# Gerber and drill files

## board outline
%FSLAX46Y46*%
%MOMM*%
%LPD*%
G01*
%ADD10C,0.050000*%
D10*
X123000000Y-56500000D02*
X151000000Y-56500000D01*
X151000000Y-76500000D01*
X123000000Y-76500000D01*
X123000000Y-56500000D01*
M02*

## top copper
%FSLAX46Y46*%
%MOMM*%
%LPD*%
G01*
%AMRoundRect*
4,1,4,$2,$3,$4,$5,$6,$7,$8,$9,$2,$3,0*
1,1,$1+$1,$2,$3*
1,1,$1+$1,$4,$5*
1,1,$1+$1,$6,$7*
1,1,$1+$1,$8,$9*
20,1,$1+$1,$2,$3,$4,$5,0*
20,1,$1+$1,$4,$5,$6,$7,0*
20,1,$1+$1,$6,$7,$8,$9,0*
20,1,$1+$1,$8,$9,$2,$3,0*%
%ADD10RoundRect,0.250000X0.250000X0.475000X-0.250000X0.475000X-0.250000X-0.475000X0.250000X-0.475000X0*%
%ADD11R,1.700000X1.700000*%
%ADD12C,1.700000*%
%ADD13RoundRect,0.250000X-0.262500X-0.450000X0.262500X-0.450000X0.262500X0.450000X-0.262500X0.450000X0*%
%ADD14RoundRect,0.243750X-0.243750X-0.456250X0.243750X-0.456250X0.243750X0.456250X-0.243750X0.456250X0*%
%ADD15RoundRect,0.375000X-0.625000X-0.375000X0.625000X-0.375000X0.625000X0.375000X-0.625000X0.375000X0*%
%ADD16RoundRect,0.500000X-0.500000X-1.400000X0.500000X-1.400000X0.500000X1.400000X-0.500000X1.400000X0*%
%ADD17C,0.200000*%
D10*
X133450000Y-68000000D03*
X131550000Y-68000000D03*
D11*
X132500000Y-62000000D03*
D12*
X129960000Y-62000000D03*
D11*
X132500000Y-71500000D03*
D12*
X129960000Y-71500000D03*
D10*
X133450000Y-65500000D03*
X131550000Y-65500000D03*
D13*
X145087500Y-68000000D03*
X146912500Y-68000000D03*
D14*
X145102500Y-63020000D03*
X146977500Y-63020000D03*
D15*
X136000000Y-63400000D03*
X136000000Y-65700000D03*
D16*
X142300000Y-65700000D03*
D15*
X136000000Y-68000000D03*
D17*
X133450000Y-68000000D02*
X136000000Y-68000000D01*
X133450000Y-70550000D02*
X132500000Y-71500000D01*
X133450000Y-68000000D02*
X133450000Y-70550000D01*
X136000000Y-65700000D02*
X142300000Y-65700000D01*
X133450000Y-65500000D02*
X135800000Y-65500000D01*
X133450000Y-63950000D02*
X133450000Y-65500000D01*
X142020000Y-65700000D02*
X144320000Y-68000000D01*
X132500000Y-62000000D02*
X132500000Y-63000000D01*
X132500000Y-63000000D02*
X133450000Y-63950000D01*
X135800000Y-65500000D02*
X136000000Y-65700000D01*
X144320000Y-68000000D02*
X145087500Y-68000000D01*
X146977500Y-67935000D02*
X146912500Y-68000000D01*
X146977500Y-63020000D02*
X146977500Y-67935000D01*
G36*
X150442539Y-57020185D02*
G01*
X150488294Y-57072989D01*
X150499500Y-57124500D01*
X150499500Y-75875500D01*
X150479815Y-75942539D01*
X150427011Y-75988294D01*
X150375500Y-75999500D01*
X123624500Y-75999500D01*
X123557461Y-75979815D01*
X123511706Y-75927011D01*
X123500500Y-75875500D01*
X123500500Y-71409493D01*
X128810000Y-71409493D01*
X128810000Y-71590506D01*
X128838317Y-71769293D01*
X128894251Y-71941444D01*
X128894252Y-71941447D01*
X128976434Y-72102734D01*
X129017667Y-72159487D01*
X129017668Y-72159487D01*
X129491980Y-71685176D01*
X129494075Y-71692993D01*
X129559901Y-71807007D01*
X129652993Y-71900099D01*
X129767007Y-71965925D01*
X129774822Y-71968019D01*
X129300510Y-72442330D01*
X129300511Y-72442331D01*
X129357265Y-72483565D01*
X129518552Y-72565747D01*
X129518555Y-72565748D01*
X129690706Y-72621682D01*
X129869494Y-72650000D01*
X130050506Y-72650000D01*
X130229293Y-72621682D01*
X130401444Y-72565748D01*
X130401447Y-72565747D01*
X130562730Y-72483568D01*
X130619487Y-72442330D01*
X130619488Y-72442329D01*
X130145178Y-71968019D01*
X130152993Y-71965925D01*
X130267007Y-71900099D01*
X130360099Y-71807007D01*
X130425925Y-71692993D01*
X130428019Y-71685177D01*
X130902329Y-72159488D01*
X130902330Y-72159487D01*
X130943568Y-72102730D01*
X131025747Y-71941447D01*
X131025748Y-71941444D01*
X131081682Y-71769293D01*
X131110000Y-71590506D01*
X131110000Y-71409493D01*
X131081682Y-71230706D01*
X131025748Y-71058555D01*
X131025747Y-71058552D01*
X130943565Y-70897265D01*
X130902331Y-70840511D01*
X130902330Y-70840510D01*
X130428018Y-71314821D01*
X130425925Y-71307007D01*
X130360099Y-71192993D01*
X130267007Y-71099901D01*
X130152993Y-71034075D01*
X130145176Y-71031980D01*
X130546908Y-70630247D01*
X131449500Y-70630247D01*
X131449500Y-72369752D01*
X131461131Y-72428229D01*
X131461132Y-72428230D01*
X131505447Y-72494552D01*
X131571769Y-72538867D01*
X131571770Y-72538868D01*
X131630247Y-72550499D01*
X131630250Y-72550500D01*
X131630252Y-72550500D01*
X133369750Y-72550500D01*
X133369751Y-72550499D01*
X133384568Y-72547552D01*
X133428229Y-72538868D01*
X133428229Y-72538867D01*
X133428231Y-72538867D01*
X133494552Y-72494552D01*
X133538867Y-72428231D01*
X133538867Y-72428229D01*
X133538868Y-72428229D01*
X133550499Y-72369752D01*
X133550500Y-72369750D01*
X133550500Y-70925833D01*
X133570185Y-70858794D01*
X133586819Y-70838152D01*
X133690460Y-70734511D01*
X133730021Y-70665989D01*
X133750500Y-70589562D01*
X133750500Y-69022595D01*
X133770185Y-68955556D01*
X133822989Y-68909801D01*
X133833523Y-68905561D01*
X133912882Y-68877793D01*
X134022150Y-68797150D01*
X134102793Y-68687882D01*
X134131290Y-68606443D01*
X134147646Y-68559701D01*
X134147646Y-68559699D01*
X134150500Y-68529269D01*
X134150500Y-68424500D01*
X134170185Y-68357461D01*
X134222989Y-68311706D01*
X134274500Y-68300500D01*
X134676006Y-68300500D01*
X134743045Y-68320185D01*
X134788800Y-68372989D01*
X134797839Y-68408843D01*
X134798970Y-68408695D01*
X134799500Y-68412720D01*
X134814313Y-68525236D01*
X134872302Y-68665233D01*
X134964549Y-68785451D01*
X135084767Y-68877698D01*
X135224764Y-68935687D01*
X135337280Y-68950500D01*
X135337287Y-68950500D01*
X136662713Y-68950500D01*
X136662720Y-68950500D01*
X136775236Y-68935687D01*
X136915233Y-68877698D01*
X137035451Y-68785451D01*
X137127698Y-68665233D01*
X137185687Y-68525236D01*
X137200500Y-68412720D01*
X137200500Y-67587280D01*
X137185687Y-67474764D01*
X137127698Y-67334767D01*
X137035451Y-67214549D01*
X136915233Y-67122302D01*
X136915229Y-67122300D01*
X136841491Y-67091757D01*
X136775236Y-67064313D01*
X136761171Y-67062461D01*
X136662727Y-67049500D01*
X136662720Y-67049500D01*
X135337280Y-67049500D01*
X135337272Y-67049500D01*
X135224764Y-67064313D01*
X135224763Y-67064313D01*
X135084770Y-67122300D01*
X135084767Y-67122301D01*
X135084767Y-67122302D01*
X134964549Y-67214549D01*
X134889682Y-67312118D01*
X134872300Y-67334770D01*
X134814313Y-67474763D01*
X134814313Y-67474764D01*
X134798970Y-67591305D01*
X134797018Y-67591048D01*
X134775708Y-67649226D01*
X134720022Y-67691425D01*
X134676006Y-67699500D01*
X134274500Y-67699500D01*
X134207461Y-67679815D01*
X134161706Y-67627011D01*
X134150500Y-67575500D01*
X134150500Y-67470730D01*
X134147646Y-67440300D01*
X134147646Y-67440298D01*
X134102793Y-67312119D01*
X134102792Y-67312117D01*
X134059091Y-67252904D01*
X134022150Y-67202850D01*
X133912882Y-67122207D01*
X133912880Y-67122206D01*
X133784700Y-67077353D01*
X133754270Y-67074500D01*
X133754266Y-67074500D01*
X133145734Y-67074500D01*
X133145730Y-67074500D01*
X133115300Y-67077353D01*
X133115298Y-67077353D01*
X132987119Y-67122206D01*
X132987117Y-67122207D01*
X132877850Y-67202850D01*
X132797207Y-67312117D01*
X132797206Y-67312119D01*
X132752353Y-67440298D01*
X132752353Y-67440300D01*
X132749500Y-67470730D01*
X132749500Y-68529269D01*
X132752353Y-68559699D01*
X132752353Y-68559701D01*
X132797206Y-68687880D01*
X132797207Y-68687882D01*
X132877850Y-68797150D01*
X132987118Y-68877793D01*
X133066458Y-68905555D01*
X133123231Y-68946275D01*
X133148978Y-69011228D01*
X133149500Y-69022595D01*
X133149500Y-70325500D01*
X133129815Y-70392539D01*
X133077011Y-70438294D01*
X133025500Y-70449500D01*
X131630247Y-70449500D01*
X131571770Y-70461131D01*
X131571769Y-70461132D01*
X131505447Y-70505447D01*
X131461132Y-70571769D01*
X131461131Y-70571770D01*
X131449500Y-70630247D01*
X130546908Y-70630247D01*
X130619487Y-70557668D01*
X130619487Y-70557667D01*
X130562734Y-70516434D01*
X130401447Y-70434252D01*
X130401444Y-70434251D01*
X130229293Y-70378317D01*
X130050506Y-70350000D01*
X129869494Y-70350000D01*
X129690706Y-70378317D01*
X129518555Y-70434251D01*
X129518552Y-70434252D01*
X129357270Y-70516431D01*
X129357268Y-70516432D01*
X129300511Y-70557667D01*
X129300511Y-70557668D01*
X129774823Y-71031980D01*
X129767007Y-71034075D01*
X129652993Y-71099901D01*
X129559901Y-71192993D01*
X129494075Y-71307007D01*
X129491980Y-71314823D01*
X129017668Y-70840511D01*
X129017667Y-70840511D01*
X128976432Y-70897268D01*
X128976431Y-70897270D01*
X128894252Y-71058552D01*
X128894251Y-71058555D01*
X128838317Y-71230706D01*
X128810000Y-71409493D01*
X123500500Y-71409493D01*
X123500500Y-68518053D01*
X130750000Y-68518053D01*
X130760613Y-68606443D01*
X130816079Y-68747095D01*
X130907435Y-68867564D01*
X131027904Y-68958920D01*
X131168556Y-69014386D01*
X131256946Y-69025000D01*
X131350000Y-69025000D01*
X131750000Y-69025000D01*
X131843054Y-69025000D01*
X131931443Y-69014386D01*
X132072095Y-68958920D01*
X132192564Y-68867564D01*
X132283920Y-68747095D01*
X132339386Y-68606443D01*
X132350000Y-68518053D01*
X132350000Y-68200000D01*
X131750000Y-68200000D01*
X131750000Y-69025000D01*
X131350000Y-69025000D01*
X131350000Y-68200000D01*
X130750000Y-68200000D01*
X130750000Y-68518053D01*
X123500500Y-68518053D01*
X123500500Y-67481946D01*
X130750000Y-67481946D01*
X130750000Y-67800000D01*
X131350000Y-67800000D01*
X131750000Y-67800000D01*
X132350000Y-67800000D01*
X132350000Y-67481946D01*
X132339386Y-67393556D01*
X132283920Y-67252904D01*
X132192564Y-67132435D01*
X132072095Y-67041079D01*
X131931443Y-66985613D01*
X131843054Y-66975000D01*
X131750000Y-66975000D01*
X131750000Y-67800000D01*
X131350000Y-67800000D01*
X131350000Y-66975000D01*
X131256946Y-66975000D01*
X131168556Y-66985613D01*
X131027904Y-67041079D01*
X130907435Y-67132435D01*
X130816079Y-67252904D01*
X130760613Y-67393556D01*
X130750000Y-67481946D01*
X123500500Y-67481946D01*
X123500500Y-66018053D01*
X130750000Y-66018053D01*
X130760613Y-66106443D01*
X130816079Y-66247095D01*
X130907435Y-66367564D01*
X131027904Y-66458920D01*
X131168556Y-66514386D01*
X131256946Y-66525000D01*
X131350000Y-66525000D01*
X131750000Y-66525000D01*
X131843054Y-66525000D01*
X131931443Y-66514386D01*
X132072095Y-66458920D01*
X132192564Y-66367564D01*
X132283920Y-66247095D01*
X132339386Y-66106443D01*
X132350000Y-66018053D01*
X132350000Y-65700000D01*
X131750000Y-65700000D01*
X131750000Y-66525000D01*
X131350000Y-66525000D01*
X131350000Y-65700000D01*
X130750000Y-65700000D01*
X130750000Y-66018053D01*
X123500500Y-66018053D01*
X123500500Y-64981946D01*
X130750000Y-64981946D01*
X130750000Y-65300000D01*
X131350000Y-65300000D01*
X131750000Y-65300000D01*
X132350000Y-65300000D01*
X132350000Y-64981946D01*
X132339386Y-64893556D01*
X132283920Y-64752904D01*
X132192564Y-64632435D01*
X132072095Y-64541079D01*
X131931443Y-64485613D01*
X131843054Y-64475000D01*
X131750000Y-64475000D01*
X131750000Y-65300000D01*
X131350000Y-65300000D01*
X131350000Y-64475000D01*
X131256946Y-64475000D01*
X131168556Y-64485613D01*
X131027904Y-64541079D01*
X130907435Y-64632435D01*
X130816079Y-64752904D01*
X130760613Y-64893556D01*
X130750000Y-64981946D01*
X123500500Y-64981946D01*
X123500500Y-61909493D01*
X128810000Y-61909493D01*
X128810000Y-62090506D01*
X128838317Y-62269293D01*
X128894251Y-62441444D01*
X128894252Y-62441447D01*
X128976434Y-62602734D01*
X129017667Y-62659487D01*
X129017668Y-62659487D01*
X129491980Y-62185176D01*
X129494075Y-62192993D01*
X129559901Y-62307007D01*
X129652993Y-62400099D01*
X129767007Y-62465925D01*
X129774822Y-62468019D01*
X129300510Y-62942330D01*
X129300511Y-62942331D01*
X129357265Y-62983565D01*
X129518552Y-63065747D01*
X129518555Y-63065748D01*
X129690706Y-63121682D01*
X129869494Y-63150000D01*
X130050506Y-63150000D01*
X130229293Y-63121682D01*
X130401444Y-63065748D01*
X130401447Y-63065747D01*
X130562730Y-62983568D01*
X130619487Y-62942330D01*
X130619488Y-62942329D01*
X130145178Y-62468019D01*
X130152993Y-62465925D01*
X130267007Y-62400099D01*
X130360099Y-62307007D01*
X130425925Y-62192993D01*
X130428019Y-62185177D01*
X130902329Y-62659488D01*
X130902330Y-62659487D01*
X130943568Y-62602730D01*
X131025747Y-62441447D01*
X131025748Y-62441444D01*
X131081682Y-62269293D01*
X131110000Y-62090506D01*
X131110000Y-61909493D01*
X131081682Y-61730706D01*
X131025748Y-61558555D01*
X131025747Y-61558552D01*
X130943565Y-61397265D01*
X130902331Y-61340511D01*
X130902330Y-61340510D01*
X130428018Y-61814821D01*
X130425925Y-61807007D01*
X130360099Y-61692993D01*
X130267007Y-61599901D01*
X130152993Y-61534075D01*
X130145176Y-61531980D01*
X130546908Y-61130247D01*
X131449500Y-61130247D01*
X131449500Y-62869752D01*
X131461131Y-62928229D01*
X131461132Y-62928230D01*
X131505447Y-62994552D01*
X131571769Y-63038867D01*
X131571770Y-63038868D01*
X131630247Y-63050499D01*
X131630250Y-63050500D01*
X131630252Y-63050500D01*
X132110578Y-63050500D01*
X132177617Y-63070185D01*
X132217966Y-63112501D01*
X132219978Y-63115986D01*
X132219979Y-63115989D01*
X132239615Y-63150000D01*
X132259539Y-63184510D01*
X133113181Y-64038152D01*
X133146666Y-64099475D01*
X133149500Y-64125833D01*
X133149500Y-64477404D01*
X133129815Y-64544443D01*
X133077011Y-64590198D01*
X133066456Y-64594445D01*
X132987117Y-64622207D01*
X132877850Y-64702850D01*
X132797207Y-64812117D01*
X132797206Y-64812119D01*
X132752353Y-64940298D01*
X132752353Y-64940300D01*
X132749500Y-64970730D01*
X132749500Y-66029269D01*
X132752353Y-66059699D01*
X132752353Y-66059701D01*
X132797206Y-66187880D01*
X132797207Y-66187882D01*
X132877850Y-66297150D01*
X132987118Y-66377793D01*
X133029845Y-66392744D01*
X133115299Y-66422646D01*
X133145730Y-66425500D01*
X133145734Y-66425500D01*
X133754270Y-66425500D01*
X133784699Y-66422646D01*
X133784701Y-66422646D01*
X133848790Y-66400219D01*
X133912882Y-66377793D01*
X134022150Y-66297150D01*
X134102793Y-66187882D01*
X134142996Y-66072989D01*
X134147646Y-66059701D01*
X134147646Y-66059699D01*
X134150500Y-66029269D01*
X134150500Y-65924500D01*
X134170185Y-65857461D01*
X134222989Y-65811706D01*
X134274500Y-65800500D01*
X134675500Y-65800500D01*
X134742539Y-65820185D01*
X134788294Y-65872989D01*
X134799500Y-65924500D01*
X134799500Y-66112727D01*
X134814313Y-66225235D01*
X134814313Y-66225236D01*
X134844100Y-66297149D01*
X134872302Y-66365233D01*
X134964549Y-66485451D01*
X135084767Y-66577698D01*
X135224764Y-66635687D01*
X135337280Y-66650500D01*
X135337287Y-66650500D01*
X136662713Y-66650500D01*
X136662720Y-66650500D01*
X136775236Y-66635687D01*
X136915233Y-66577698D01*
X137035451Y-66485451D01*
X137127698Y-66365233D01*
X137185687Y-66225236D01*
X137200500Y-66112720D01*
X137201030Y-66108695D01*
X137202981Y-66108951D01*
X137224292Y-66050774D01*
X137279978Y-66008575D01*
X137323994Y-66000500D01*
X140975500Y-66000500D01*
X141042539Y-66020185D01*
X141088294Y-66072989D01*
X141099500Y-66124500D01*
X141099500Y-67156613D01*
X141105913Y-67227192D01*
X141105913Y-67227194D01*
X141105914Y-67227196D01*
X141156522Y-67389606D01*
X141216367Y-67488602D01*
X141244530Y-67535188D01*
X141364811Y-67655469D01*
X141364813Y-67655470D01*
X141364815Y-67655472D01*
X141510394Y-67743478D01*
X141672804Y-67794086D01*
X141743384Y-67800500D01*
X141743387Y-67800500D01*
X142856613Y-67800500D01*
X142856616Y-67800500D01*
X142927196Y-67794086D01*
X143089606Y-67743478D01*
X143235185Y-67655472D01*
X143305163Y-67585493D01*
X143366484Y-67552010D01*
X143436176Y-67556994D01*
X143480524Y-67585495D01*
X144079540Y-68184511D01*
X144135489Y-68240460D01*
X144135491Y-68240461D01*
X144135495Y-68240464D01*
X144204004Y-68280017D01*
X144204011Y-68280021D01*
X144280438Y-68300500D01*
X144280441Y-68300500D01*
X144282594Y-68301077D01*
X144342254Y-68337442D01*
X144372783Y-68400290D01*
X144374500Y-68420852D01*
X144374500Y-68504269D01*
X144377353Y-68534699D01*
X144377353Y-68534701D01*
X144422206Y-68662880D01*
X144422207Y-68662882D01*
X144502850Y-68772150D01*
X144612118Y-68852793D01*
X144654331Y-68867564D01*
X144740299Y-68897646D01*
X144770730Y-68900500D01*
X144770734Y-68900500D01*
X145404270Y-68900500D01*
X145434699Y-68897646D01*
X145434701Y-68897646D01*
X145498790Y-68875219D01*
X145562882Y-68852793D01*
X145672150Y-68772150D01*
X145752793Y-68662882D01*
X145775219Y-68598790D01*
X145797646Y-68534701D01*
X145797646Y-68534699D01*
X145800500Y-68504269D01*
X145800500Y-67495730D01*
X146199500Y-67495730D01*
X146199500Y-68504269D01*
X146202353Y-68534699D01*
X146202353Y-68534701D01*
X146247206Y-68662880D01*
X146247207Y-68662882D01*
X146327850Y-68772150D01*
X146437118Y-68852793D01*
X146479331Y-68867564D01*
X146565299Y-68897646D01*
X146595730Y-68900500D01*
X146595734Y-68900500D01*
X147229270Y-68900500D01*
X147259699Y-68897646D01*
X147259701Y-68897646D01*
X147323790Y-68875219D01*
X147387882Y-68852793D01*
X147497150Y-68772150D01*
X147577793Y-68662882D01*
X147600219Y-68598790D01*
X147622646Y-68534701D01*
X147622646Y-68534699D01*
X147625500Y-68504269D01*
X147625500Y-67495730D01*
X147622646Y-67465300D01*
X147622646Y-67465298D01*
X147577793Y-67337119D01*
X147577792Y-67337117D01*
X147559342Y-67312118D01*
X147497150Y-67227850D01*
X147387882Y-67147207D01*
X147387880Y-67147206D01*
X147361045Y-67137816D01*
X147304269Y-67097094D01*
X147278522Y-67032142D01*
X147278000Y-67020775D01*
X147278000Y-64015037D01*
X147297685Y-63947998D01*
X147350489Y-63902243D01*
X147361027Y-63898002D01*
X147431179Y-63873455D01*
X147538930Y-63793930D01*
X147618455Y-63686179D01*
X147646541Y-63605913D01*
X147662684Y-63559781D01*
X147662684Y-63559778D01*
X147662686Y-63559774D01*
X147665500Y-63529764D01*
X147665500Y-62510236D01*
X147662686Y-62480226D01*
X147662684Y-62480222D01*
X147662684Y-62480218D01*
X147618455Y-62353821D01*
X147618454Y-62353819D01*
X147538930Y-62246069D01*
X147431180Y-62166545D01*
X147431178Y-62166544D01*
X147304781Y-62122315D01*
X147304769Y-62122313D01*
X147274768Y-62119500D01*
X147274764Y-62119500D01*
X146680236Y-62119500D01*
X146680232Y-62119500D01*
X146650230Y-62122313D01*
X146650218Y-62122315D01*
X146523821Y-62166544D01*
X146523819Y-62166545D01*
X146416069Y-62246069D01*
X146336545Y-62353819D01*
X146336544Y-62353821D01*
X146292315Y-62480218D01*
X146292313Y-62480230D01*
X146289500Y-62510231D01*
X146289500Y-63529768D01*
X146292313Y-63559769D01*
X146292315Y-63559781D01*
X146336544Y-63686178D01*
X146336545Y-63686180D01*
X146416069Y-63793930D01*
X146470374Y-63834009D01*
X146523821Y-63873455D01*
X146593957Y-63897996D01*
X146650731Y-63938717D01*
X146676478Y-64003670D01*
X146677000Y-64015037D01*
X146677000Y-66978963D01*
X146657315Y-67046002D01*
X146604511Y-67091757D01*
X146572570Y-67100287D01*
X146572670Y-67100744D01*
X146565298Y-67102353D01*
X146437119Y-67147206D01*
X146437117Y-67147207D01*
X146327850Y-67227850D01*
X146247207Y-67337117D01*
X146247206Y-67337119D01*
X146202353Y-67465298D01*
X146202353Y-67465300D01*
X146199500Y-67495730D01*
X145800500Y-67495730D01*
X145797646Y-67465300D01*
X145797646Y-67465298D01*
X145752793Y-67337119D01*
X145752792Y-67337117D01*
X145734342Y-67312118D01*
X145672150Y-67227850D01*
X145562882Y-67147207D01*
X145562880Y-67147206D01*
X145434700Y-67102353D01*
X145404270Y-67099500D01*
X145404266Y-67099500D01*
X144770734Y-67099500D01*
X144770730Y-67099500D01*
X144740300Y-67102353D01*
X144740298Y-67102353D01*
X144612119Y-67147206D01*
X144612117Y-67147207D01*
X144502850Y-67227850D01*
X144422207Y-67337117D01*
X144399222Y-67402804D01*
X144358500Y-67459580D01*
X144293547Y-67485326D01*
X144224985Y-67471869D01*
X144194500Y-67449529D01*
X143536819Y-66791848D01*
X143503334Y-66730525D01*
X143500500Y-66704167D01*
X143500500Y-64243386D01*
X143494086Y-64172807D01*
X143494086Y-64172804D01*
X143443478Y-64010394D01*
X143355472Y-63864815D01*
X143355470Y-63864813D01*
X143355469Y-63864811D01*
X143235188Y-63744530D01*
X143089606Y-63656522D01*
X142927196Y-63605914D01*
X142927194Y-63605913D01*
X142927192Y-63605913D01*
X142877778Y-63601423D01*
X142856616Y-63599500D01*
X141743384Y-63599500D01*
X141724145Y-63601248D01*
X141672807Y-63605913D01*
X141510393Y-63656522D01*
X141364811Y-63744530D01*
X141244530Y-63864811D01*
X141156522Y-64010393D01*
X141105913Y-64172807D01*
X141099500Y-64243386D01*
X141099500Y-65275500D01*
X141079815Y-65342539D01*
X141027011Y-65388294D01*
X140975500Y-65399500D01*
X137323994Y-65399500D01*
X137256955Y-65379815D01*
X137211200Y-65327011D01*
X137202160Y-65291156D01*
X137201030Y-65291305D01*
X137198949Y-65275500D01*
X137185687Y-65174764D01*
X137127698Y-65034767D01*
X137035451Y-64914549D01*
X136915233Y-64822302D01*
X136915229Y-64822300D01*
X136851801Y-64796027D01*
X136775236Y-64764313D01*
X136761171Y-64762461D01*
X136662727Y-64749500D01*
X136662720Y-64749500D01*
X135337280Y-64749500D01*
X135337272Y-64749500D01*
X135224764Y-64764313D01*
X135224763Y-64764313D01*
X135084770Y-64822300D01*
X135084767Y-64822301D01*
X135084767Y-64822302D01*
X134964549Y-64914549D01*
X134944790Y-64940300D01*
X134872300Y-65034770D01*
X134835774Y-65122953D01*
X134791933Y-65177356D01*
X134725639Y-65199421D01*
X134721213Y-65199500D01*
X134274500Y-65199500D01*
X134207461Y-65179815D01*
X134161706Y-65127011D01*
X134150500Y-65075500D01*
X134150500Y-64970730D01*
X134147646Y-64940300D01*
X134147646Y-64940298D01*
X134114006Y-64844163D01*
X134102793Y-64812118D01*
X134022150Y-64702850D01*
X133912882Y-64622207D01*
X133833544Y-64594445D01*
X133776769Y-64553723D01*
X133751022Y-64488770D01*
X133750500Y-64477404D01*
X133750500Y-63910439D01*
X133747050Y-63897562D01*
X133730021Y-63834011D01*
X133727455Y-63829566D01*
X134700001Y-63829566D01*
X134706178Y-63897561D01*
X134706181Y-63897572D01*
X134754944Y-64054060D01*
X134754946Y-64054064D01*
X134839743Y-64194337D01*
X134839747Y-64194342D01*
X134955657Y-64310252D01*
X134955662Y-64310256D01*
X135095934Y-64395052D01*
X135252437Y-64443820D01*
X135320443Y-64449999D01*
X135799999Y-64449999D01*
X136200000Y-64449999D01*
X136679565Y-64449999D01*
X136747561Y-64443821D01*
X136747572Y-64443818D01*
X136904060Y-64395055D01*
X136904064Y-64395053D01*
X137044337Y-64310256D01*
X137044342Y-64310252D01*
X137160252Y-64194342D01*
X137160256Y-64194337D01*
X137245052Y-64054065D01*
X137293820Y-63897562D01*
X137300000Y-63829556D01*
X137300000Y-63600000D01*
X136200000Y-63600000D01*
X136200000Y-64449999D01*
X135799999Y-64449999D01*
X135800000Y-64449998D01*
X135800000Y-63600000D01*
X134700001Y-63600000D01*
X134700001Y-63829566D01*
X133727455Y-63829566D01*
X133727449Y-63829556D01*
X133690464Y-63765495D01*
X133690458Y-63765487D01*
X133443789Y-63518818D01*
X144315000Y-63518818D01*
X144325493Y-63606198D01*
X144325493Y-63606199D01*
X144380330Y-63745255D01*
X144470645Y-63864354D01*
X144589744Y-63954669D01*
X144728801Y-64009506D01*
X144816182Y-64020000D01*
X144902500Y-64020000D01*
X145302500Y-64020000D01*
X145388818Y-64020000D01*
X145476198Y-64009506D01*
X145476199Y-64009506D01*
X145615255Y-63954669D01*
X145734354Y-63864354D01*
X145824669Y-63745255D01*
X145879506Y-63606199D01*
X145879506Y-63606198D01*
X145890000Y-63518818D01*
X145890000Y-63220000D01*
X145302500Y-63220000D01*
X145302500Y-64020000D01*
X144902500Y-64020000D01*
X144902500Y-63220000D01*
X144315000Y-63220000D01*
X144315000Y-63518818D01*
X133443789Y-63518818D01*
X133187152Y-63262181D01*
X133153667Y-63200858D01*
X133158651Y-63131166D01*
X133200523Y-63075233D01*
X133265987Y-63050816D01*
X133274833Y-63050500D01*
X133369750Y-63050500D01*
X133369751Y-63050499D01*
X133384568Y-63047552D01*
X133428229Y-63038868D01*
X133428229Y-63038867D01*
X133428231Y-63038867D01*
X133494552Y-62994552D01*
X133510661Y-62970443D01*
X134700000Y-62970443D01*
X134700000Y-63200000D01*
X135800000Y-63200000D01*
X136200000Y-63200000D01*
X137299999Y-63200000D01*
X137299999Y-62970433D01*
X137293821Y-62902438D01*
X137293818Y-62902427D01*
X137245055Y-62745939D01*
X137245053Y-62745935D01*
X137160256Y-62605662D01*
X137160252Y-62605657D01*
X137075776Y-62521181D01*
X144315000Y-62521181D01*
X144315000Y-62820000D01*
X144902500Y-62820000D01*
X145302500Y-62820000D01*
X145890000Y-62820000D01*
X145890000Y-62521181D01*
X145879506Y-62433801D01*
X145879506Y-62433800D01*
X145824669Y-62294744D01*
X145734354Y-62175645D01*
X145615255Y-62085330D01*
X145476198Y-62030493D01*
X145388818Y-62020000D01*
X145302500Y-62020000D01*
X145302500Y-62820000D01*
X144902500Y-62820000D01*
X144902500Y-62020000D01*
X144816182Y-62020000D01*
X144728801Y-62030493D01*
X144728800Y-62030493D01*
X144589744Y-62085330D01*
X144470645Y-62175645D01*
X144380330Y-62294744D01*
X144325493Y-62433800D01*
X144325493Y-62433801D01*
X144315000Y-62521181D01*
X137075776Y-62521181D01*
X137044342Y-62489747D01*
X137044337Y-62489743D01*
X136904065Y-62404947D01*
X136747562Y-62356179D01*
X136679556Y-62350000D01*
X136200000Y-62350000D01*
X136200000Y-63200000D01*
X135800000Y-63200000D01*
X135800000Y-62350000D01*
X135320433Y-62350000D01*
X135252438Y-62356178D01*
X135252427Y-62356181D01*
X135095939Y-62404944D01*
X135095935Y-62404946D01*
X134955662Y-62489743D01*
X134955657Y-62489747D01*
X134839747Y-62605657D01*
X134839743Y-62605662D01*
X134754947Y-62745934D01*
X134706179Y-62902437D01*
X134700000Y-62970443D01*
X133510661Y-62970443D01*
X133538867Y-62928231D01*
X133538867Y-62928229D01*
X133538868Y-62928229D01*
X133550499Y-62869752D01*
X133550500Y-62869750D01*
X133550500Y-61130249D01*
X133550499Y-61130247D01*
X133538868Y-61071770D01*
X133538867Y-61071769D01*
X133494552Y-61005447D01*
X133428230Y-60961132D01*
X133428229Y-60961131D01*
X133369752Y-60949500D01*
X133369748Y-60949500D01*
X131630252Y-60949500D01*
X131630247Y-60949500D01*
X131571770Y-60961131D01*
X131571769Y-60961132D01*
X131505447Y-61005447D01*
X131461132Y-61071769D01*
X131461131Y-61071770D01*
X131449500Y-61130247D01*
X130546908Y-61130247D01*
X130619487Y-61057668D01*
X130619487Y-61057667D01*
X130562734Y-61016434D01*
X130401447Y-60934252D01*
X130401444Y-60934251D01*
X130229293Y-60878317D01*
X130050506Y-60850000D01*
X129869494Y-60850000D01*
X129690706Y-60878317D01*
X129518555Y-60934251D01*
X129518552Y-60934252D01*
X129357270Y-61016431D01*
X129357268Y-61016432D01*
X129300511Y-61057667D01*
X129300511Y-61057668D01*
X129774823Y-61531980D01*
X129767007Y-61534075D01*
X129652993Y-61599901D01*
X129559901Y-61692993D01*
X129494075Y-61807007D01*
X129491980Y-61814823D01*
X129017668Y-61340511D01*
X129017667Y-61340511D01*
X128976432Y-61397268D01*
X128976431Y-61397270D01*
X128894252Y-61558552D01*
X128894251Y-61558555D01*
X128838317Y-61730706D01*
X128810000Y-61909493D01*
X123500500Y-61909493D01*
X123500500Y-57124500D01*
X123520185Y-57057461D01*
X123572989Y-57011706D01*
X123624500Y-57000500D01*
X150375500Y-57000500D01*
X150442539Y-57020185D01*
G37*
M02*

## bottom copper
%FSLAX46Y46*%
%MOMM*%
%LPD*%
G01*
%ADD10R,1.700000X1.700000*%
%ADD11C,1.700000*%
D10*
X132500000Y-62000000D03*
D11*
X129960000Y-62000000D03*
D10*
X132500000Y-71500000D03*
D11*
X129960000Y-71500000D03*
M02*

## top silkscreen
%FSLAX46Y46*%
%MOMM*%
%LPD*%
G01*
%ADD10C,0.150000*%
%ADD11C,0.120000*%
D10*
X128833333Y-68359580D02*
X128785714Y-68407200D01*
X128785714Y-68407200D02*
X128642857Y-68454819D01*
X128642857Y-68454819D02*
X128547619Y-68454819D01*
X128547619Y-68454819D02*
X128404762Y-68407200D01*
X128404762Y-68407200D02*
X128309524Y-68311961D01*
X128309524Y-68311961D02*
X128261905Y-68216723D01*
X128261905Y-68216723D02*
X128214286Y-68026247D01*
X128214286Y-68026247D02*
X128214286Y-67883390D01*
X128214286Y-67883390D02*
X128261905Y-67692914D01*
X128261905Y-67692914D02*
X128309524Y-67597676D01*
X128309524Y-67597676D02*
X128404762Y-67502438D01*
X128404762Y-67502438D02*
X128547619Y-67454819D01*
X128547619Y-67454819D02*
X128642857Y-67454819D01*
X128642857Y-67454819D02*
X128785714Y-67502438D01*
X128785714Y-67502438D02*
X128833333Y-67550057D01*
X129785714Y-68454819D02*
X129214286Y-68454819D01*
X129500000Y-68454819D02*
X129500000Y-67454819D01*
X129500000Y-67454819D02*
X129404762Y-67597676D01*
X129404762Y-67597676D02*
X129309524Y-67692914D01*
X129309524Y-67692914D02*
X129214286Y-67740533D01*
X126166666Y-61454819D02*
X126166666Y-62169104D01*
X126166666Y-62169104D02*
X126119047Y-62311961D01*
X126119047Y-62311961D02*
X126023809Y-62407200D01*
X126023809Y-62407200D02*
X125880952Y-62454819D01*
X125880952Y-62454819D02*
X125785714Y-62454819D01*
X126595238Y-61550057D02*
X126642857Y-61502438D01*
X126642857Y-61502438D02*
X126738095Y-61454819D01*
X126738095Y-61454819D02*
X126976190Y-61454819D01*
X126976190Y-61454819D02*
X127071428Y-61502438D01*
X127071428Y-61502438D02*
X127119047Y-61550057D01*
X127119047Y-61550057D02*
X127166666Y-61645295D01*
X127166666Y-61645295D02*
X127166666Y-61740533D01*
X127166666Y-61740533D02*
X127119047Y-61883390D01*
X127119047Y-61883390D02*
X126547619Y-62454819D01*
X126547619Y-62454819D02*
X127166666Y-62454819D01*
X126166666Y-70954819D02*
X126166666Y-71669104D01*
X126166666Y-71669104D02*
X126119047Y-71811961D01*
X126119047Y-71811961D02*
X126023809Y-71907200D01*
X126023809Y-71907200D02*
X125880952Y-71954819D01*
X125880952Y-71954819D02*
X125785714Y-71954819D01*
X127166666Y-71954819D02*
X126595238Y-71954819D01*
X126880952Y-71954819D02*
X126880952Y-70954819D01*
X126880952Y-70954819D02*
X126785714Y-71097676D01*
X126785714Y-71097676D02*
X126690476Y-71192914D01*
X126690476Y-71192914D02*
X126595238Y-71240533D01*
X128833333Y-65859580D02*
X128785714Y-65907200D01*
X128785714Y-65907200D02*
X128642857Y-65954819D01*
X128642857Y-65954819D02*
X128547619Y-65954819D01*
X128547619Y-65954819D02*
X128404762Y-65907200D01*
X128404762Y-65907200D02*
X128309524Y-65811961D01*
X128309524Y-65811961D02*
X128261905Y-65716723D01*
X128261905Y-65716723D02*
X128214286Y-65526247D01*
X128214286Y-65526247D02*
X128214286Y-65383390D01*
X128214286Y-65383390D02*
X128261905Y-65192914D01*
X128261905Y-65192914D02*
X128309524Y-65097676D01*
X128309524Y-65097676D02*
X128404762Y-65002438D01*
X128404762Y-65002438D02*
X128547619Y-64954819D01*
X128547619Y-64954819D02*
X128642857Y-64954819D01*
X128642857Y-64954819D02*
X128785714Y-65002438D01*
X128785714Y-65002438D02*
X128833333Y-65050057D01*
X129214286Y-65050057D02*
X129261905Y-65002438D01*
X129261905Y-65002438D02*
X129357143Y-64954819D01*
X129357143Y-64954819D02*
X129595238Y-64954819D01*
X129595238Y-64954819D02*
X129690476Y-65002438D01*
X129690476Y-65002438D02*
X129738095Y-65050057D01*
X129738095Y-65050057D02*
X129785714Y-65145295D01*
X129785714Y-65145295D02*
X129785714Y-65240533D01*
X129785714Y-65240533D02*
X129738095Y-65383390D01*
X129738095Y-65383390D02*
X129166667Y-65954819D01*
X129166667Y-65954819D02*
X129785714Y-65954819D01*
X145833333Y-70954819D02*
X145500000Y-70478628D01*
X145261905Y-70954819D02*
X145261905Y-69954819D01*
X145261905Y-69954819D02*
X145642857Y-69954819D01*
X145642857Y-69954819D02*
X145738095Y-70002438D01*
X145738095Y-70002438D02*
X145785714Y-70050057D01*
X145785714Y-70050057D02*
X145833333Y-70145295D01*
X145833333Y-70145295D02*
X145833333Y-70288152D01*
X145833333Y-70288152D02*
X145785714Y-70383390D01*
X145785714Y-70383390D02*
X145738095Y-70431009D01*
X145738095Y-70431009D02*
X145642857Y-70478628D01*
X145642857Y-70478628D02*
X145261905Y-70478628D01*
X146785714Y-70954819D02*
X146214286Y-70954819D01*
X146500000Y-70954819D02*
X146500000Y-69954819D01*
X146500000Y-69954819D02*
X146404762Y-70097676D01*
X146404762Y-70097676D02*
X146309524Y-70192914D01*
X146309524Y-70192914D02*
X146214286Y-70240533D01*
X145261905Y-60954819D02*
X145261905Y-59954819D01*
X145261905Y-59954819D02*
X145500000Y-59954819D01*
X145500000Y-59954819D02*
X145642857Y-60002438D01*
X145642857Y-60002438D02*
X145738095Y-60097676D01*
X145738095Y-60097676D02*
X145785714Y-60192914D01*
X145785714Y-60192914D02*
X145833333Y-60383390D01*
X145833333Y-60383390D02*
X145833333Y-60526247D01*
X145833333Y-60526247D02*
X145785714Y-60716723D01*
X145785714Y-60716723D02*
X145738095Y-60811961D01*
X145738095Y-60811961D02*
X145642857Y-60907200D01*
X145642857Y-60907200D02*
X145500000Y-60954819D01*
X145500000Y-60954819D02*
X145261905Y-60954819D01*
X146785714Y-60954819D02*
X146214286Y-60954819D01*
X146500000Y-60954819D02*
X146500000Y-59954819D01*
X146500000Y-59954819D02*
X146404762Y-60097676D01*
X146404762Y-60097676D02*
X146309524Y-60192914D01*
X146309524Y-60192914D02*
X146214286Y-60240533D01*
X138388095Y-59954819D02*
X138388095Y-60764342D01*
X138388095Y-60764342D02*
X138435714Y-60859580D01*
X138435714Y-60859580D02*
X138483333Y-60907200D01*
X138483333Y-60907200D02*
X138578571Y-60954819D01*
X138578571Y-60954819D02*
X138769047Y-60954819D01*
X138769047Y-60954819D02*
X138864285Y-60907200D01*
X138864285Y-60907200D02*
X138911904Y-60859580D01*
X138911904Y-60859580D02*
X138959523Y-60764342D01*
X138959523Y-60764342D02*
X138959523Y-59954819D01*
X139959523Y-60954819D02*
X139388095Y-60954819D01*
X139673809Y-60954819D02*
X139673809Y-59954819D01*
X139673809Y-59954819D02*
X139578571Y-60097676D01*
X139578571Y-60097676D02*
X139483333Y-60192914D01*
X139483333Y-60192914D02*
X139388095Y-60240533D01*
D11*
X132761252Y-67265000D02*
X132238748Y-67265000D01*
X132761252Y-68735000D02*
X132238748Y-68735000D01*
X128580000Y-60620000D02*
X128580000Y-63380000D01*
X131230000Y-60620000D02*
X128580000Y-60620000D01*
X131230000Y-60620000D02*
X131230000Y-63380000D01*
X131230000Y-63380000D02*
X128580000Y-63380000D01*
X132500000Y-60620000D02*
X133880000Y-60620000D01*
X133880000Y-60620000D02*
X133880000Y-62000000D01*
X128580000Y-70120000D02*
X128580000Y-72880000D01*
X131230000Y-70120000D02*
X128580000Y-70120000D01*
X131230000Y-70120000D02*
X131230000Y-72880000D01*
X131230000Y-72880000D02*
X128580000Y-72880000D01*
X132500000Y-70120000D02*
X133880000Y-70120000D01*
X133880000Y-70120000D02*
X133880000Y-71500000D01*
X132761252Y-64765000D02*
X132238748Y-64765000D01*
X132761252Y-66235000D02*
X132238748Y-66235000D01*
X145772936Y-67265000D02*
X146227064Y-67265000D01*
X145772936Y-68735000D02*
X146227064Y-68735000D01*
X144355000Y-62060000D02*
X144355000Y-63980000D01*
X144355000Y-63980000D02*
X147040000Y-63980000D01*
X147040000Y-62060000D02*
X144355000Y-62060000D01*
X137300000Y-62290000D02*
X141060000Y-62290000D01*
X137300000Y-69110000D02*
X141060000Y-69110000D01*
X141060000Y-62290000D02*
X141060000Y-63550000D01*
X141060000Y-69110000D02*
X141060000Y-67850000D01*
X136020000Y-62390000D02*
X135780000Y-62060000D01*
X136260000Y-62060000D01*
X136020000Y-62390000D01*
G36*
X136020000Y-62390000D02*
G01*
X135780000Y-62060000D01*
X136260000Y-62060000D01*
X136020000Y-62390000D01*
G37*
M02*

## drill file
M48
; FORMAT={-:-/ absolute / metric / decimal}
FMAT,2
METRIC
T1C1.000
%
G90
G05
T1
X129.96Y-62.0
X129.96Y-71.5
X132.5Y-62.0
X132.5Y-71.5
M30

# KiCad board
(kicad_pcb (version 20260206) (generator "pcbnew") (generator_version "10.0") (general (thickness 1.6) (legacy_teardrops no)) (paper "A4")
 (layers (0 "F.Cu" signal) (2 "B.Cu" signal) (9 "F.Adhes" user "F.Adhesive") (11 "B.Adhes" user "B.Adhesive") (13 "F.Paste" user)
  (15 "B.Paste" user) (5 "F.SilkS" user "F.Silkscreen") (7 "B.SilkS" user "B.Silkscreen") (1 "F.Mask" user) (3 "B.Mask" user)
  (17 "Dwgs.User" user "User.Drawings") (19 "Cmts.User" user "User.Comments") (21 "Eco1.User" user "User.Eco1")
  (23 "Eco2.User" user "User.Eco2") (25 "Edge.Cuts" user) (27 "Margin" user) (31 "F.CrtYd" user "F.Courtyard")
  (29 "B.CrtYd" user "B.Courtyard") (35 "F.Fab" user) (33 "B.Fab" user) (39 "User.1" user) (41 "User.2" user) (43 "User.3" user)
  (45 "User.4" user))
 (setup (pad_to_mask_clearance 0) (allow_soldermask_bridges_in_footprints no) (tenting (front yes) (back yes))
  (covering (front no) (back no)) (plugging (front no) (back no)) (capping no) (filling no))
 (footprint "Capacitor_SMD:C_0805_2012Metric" (layer "F.Cu") (at 132.5 68 180)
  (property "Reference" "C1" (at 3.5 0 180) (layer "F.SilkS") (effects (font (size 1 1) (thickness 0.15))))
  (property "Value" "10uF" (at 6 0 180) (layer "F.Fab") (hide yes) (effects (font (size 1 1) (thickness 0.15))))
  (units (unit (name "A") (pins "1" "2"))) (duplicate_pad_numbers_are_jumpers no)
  (fp_line (start -0.261252 0.735) (end 0.261252 0.735) (stroke (width 0.12) (type solid)) (layer "F.SilkS"))
  (fp_line (start -0.261252 -0.735) (end 0.261252 -0.735) (stroke (width 0.12) (type solid)) (layer "F.SilkS"))
  (pad "1" smd roundrect (at -0.95 0 180) (size 1 1.45) (layers "F.Cu" "F.Mask" "F.Paste") (roundrect_rratio 0.25) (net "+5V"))
  (pad "2" smd roundrect (at 0.95 0 180) (size 1 1.45) (layers "F.Cu" "F.Mask" "F.Paste") (roundrect_rratio 0.25) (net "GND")))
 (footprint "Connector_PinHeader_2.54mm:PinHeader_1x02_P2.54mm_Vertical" (layer "F.Cu") (at 132.5 62 -90)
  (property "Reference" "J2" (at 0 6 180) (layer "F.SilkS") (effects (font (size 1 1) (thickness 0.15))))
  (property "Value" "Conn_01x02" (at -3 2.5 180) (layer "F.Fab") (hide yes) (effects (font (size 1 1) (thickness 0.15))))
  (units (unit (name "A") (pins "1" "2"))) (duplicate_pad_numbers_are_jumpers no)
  (fp_line (start -1.38 3.92) (end 1.38 3.92) (stroke (width 0.12) (type solid)) (layer "F.SilkS"))
  (fp_line (start -1.38 1.27) (end -1.38 3.92) (stroke (width 0.12) (type solid)) (layer "F.SilkS"))
  (fp_line (start -1.38 1.27) (end 1.38 1.27) (stroke (width 0.12) (type solid)) (layer "F.SilkS"))
  (fp_line (start 1.38 1.27) (end 1.38 3.92) (stroke (width 0.12) (type solid)) (layer "F.SilkS"))
  (fp_line (start -1.38 0) (end -1.38 -1.38) (stroke (width 0.12) (type solid)) (layer "F.SilkS"))
  (fp_line (start -1.38 -1.38) (end 0 -1.38) (stroke (width 0.12) (type solid)) (layer "F.SilkS"))
  (pad "1" thru_hole rect (at 0 0 270) (size 1.7 1.7) (drill 1) (layers "*.Cu" "*.Mask") (remove_unused_layers no) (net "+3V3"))
  (pad "2" thru_hole circle (at 0 2.54 270) (size 1.7 1.7) (drill 1) (layers "*.Cu" "*.Mask") (remove_unused_layers no) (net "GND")))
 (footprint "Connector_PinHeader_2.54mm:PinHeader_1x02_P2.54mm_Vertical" (layer "F.Cu") (at 132.5 71.5 -90)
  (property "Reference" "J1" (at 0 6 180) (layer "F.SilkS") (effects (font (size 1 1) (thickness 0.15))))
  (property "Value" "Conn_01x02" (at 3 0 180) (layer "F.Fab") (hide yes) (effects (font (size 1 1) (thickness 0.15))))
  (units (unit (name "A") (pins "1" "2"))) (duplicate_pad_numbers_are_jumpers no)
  (fp_line (start -1.38 3.92) (end 1.38 3.92) (stroke (width 0.12) (type solid)) (layer "F.SilkS"))
  (fp_line (start -1.38 1.27) (end -1.38 3.92) (stroke (width 0.12) (type solid)) (layer "F.SilkS"))
  (fp_line (start -1.38 1.27) (end 1.38 1.27) (stroke (width 0.12) (type solid)) (layer "F.SilkS"))
  (fp_line (start 1.38 1.27) (end 1.38 3.92) (stroke (width 0.12) (type solid)) (layer "F.SilkS"))
  (fp_line (start -1.38 0) (end -1.38 -1.38) (stroke (width 0.12) (type solid)) (layer "F.SilkS"))
  (fp_line (start -1.38 -1.38) (end 0 -1.38) (stroke (width 0.12) (type solid)) (layer "F.SilkS"))
  (pad "1" thru_hole rect (at 0 0 270) (size 1.7 1.7) (drill 1) (layers "*.Cu" "*.Mask") (remove_unused_layers no) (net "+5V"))
  (pad "2" thru_hole circle (at 0 2.54 270) (size 1.7 1.7) (drill 1) (layers "*.Cu" "*.Mask") (remove_unused_layers no) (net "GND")))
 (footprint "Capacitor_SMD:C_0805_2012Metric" (layer "F.Cu") (at 132.5 65.5 180)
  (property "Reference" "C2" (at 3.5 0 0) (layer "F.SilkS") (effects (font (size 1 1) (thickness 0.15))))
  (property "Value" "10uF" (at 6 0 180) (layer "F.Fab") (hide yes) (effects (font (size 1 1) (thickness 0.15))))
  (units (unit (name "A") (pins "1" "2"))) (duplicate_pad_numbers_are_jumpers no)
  (fp_line (start -0.261252 0.735) (end 0.261252 0.735) (stroke (width 0.12) (type solid)) (layer "F.SilkS"))
  (fp_line (start -0.261252 -0.735) (end 0.261252 -0.735) (stroke (width 0.12) (type solid)) (layer "F.SilkS"))
  (pad "1" smd roundrect (at -0.95 0 180) (size 1 1.45) (layers "F.Cu" "F.Mask" "F.Paste") (roundrect_rratio 0.25) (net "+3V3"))
  (pad "2" smd roundrect (at 0.95 0 180) (size 1 1.45) (layers "F.Cu" "F.Mask" "F.Paste") (roundrect_rratio 0.25) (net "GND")))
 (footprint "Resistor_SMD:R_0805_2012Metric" (layer "F.Cu") (at 146 68)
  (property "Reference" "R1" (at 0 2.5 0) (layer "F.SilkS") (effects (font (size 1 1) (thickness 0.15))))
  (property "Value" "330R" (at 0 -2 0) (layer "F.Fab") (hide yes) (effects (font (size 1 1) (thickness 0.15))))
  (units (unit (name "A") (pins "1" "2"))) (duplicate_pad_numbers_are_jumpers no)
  (fp_line (start -0.227064 -0.735) (end 0.227064 -0.735) (stroke (width 0.12) (type solid)) (layer "F.SilkS"))
  (fp_line (start -0.227064 0.735) (end 0.227064 0.735) (stroke (width 0.12) (type solid)) (layer "F.SilkS"))
  (pad "1" smd roundrect (at -0.9125 0) (size 1.025 1.4) (layers "F.Cu" "F.Mask" "F.Paste") (roundrect_rratio 0.243902) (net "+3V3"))
  (pad "2" smd roundrect (at 0.9125 0) (size 1.025 1.4) (layers "F.Cu" "F.Mask" "F.Paste") (roundrect_rratio 0.243902) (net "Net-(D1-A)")))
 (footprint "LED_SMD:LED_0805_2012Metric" (layer "F.Cu") (at 146.04 63.02)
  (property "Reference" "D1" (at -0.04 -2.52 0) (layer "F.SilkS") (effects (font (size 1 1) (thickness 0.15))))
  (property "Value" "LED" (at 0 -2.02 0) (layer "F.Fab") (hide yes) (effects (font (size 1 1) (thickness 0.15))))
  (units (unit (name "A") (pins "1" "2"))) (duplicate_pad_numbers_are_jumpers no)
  (fp_line (start -1.685 -0.96) (end -1.685 0.96) (stroke (width 0.12) (type solid)) (layer "F.SilkS"))
  (fp_line (start -1.685 0.96) (end 1 0.96) (stroke (width 0.12) (type solid)) (layer "F.SilkS"))
  (fp_line (start 1 -0.96) (end -1.685 -0.96) (stroke (width 0.12) (type solid)) (layer "F.SilkS"))
  (pad "1" smd roundrect (at -0.9375 0) (size 0.975 1.4) (layers "F.Cu" "F.Mask" "F.Paste") (roundrect_rratio 0.25) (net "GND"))
  (pad "2" smd roundrect (at 0.9375 0) (size 0.975 1.4) (layers "F.Cu" "F.Mask" "F.Paste") (roundrect_rratio 0.25) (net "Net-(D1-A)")))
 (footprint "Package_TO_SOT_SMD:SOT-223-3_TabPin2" (layer "F.Cu") (at 139.15 65.7)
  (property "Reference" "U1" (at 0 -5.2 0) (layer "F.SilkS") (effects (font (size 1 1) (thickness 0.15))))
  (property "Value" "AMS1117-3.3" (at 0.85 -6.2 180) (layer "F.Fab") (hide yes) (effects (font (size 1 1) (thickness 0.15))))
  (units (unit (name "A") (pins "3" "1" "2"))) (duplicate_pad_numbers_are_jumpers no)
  (fp_line (start -1.85 -3.41) (end 1.91 -3.41) (stroke (width 0.12) (type solid)) (layer "F.SilkS"))
  (fp_line (start -1.85 3.41) (end 1.91 3.41) (stroke (width 0.12) (type solid)) (layer "F.SilkS"))
  (fp_line (start 1.91 -3.41) (end 1.91 -2.15) (stroke (width 0.12) (type solid)) (layer "F.SilkS"))
  (fp_line (start 1.91 3.41) (end 1.91 2.15) (stroke (width 0.12) (type solid)) (layer "F.SilkS"))
  (fp_poly
   (pts (xy -3.13 -3.31) (xy -3.37 -3.64) (xy -2.89 -3.64) (xy -3.13 -3.31)) (stroke (width 0.12) (type solid)) (fill yes) (layer "F.SilkS"))
  (pad "1" smd roundrect (at -3.15 -2.3) (size 2 1.5) (layers "F.Cu" "F.Mask" "F.Paste") (roundrect_rratio 0.25) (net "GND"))
  (pad "2" smd roundrect (at -3.15 0) (size 2 1.5) (layers "F.Cu" "F.Mask" "F.Paste") (roundrect_rratio 0.25) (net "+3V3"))
  (pad "2" smd roundrect (at 3.15 0) (size 2 3.8) (layers "F.Cu" "F.Mask" "F.Paste") (roundrect_rratio 0.25) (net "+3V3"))
  (pad "3" smd roundrect (at -3.15 2.3) (size 2 1.5) (layers "F.Cu" "F.Mask" "F.Paste") (roundrect_rratio 0.25) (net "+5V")))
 (gr_rect (start 123 56.5) (end 151 76.5) (stroke (width 0.05) (type default)) (fill no) (layer "Edge.Cuts"))
 (segment (start 133.45 68) (end 136 68) (width 0.2) (layer "F.Cu") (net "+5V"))
 (segment (start 133.45 70.55) (end 132.5 71.5) (width 0.2) (layer "F.Cu") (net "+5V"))
 (segment (start 133.45 68) (end 133.45 70.55) (width 0.2) (layer "F.Cu") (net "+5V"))
 (segment (start 136 65.7) (end 142.3 65.7) (width 0.2) (layer "F.Cu") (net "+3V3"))
 (segment (start 133.45 65.5) (end 135.8 65.5) (width 0.2) (layer "F.Cu") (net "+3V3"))
 (segment (start 133.45 63.95) (end 133.45 65.5) (width 0.2) (layer "F.Cu") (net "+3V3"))
 (segment (start 142.02 65.7) (end 144.32 68) (width 0.2) (layer "F.Cu") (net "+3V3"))
 (segment (start 132.5 62) (end 132.5 63) (width 0.2) (layer "F.Cu") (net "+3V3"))
 (segment (start 132.5 63) (end 133.45 63.95) (width 0.2) (layer "F.Cu") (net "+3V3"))
 (segment (start 135.8 65.5) (end 136 65.7) (width 0.2) (layer "F.Cu") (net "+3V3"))
 (segment (start 144.32 68) (end 145.0875 68) (width 0.2) (layer "F.Cu") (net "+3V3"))
 (segment (start 146.9775 67.935) (end 146.9125 68) (width 0.2) (layer "F.Cu") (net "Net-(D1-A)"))
 (segment (start 146.9775 63.02) (end 146.9775 67.935) (width 0.2) (layer "F.Cu") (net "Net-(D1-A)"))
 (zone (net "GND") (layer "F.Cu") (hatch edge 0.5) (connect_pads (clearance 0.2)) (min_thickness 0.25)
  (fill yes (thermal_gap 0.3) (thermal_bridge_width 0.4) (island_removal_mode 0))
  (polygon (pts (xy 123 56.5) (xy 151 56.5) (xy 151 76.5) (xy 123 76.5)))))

